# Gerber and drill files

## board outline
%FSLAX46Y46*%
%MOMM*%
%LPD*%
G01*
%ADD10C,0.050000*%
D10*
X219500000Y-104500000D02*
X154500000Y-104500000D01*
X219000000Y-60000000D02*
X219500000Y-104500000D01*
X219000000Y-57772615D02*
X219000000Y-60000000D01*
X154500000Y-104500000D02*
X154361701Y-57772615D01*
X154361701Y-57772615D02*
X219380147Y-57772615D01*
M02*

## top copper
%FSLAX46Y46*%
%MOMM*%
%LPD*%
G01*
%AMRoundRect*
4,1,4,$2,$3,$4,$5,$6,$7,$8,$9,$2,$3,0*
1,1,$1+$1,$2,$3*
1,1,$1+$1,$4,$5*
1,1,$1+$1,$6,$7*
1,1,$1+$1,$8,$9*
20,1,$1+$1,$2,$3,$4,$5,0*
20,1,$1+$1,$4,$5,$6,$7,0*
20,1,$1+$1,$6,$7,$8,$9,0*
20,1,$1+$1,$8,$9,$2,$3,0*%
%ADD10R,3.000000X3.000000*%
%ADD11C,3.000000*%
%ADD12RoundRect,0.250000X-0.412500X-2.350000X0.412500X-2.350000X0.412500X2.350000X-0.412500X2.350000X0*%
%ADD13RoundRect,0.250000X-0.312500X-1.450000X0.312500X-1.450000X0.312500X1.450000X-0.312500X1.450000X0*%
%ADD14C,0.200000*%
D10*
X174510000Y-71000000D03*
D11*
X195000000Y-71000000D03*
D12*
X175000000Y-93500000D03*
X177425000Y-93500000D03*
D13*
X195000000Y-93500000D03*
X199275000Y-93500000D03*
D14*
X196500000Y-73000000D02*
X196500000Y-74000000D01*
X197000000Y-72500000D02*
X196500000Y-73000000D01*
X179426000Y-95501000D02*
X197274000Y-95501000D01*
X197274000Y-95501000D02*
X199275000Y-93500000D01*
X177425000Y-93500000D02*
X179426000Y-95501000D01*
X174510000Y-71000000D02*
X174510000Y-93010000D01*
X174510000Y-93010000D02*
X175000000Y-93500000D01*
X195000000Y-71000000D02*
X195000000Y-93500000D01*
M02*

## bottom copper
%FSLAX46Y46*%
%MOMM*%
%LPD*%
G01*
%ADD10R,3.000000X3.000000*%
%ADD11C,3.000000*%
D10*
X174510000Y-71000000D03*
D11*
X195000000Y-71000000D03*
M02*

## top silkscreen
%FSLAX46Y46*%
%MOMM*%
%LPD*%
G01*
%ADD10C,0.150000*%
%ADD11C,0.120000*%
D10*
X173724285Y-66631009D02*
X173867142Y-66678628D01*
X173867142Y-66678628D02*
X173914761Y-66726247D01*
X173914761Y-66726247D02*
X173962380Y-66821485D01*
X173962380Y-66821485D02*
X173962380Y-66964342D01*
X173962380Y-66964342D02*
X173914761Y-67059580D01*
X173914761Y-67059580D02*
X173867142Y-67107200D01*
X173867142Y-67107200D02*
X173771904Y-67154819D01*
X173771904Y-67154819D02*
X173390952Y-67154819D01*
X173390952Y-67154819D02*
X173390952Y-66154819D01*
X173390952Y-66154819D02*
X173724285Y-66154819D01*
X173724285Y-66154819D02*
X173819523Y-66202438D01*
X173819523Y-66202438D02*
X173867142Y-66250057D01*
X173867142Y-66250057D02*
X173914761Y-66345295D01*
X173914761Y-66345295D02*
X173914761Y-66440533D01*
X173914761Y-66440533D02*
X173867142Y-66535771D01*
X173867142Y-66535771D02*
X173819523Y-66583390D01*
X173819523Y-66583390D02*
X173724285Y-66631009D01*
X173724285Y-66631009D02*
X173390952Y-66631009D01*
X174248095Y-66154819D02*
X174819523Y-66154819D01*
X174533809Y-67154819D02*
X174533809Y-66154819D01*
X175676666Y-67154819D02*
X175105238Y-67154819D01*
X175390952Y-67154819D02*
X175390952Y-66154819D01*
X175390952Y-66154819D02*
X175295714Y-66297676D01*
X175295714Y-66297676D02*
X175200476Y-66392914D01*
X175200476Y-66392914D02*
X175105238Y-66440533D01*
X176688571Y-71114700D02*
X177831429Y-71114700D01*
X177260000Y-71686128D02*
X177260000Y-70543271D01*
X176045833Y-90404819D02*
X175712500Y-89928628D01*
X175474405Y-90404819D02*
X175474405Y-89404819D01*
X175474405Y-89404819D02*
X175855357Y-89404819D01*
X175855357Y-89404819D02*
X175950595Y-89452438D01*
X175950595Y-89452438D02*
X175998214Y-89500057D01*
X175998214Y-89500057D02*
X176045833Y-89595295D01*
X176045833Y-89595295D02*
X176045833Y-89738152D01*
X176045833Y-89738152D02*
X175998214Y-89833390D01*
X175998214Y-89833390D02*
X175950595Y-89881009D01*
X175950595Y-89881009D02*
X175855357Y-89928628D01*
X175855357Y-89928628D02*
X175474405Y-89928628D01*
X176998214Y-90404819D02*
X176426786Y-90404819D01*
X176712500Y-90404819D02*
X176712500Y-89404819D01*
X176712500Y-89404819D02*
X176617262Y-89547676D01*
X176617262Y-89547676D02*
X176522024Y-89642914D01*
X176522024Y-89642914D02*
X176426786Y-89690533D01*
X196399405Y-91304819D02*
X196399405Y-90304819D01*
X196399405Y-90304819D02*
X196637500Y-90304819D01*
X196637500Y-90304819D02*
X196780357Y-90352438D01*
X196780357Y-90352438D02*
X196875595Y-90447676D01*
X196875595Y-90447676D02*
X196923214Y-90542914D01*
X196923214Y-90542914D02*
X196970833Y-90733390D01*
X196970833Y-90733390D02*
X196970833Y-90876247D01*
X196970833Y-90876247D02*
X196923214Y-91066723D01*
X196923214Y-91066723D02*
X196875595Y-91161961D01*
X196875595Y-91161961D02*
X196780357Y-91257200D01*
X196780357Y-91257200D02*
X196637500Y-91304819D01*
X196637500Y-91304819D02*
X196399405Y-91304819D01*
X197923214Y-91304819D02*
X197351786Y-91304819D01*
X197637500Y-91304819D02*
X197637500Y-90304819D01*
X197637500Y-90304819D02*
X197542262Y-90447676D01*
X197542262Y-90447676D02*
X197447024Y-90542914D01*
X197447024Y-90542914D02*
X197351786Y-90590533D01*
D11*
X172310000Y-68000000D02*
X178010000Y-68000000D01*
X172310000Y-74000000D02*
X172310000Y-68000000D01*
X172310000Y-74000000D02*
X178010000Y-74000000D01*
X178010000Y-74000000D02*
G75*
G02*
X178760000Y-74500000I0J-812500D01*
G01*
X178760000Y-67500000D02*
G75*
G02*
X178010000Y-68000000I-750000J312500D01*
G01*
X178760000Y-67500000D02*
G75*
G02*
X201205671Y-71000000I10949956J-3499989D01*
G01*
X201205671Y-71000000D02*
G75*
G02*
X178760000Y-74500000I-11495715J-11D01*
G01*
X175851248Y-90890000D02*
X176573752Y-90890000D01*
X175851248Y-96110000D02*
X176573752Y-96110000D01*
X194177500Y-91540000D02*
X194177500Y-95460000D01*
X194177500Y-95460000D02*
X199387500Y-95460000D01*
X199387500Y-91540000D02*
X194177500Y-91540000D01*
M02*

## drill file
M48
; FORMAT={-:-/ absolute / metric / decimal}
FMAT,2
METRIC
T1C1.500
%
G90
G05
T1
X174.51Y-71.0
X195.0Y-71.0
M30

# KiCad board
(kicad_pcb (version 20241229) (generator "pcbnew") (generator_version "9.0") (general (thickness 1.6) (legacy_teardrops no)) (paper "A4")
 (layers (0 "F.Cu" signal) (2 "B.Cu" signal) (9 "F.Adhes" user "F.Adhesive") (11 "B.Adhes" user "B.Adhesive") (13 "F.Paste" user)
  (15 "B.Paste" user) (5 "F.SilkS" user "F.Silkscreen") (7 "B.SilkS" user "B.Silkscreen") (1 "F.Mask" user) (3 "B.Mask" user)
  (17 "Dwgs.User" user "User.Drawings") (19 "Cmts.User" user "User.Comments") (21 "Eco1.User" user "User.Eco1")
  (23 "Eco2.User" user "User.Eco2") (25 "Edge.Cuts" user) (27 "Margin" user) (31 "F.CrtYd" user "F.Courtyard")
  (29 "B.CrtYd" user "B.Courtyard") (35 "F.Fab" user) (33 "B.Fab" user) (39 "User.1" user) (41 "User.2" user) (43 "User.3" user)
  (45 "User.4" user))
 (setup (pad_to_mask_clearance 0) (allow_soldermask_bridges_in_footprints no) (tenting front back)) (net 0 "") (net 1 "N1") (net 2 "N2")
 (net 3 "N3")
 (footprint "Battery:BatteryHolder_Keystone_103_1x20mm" (layer "F.Cu") (at 174.51 71)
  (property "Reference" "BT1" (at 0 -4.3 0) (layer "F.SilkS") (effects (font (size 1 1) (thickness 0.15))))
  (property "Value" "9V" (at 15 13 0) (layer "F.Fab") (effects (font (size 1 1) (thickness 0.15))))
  (fp_line (start -2.2 -3) (end 3.5 -3) (stroke (width 0.12) (type solid)) (layer "F.SilkS"))
  (fp_line (start -2.2 3) (end -2.2 -3) (stroke (width 0.12) (type solid)) (layer "F.SilkS"))
  (fp_line (start -2.2 3) (end 3.5 3) (stroke (width 0.12) (type solid)) (layer "F.SilkS"))
  (fp_arc (start 3.5 3) (mid 3.950694 3.136459) (end 4.25 3.5) (stroke (width 0.12) (type solid)) (layer "F.SilkS"))
  (fp_arc (start 4.25 -3.5) (mid 3.950694 -3.136459) (end 3.5 -3) (stroke (width 0.12) (type solid)) (layer "F.SilkS"))
  (fp_arc (start 4.25 -3.5) (mid 16.971103 -11.358466) (end 26.695671 0) (stroke (width 0.12) (type solid)) (layer "F.SilkS"))
  (fp_arc (start 26.695671 0) (mid 16.971103 11.358466) (end 4.25 3.5) (stroke (width 0.12) (type solid)) (layer "F.SilkS"))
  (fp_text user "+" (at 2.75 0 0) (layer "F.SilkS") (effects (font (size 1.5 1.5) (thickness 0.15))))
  (pad "1" thru_hole rect (at 0 0) (size 3 3) (drill 1.5) (layers "*.Cu" "*.Mask") (remove_unused_layers no) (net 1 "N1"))
  (pad "2" thru_hole circle (at 20.49 0) (size 3 3) (drill 1.5) (layers "*.Cu" "*.Mask") (remove_unused_layers no) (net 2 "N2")))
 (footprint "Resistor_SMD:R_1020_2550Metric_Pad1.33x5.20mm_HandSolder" (layer "F.Cu") (at 176.2125 93.5)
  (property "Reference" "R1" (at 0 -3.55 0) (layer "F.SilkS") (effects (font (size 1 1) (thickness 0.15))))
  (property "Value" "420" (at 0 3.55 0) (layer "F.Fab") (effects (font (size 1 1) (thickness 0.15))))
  (fp_line (start -0.361252 -2.61) (end 0.361252 -2.61) (stroke (width 0.12) (type solid)) (layer "F.SilkS"))
  (fp_line (start -0.361252 2.61) (end 0.361252 2.61) (stroke (width 0.12) (type solid)) (layer "F.SilkS"))
  (pad "1" smd roundrect (at -1.2125 0) (size 1.325 5.2) (layers "F.Cu" "F.Mask" "F.Paste") (roundrect_rratio 0.188679) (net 1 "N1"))
  (pad "2" smd roundrect (at 1.2125 0) (size 1.325 5.2) (layers "F.Cu" "F.Mask" "F.Paste") (roundrect_rratio 0.188679) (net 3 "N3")))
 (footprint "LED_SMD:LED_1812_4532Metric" (layer "F.Cu") (at 197.1375 93.5)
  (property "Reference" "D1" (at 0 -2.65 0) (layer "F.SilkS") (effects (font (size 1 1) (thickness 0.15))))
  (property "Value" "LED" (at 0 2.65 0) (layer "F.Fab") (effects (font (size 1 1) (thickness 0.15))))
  (fp_line (start -2.96 -1.96) (end -2.96 1.96) (stroke (width 0.12) (type solid)) (layer "F.SilkS"))
  (fp_line (start -2.96 1.96) (end 2.25 1.96) (stroke (width 0.12) (type solid)) (layer "F.SilkS"))
  (fp_line (start 2.25 -1.96) (end -2.96 -1.96) (stroke (width 0.12) (type solid)) (layer "F.SilkS"))
  (pad "1" smd roundrect (at -2.1375 0) (size 1.125 3.4) (layers "F.Cu" "F.Mask" "F.Paste") (roundrect_rratio 0.222222) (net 2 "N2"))
  (pad "2" smd roundrect (at 2.1375 0) (size 1.125 3.4) (layers "F.Cu" "F.Mask" "F.Paste") (roundrect_rratio 0.222222) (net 3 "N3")))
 (gr_line (start 219.5 104.5) (end 154.5 104.5) (stroke (width 0.05) (type default)) (layer "Edge.Cuts"))
 (gr_line (start 219 60) (end 219.5 104.5) (stroke (width 0.05) (type default)) (layer "Edge.Cuts"))
 (gr_line (start 219 57.772615) (end 219 60) (stroke (width 0.05) (type default)) (layer "Edge.Cuts"))
 (gr_line (start 154.5 104.5) (end 154.361701 57.772615) (stroke (width 0.05) (type default)) (layer "Edge.Cuts"))
 (gr_line (start 154.361701 57.772615) (end 219.380147 57.772615) (stroke (width 0.05) (type default)) (layer "Edge.Cuts"))
 (segment (start 196.5 73) (end 196.5 74) (width 0.2) (layer "F.Cu") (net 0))
 (segment (start 197 72.5) (end 196.5 73) (width 0.2) (layer "F.Cu") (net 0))
 (segment (start 179.426 95.501) (end 197.274 95.501) (width 0.2) (layer "F.Cu") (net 3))
 (segment (start 197.274 95.501) (end 199.275 93.5) (width 0.2) (layer "F.Cu") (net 3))
 (segment (start 177.425 93.5) (end 179.426 95.501) (width 0.2) (layer "F.Cu") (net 3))
 (segment (start 174.51 71) (end 174.51 93.01) (width 0.2) (layer "F.Cu") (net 1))
 (segment (start 174.51 93.01) (end 175 93.5) (width 0.2) (layer "F.Cu") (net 1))
 (segment (start 195 71) (end 195 93.5) (width 0.2) (layer "F.Cu") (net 2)))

